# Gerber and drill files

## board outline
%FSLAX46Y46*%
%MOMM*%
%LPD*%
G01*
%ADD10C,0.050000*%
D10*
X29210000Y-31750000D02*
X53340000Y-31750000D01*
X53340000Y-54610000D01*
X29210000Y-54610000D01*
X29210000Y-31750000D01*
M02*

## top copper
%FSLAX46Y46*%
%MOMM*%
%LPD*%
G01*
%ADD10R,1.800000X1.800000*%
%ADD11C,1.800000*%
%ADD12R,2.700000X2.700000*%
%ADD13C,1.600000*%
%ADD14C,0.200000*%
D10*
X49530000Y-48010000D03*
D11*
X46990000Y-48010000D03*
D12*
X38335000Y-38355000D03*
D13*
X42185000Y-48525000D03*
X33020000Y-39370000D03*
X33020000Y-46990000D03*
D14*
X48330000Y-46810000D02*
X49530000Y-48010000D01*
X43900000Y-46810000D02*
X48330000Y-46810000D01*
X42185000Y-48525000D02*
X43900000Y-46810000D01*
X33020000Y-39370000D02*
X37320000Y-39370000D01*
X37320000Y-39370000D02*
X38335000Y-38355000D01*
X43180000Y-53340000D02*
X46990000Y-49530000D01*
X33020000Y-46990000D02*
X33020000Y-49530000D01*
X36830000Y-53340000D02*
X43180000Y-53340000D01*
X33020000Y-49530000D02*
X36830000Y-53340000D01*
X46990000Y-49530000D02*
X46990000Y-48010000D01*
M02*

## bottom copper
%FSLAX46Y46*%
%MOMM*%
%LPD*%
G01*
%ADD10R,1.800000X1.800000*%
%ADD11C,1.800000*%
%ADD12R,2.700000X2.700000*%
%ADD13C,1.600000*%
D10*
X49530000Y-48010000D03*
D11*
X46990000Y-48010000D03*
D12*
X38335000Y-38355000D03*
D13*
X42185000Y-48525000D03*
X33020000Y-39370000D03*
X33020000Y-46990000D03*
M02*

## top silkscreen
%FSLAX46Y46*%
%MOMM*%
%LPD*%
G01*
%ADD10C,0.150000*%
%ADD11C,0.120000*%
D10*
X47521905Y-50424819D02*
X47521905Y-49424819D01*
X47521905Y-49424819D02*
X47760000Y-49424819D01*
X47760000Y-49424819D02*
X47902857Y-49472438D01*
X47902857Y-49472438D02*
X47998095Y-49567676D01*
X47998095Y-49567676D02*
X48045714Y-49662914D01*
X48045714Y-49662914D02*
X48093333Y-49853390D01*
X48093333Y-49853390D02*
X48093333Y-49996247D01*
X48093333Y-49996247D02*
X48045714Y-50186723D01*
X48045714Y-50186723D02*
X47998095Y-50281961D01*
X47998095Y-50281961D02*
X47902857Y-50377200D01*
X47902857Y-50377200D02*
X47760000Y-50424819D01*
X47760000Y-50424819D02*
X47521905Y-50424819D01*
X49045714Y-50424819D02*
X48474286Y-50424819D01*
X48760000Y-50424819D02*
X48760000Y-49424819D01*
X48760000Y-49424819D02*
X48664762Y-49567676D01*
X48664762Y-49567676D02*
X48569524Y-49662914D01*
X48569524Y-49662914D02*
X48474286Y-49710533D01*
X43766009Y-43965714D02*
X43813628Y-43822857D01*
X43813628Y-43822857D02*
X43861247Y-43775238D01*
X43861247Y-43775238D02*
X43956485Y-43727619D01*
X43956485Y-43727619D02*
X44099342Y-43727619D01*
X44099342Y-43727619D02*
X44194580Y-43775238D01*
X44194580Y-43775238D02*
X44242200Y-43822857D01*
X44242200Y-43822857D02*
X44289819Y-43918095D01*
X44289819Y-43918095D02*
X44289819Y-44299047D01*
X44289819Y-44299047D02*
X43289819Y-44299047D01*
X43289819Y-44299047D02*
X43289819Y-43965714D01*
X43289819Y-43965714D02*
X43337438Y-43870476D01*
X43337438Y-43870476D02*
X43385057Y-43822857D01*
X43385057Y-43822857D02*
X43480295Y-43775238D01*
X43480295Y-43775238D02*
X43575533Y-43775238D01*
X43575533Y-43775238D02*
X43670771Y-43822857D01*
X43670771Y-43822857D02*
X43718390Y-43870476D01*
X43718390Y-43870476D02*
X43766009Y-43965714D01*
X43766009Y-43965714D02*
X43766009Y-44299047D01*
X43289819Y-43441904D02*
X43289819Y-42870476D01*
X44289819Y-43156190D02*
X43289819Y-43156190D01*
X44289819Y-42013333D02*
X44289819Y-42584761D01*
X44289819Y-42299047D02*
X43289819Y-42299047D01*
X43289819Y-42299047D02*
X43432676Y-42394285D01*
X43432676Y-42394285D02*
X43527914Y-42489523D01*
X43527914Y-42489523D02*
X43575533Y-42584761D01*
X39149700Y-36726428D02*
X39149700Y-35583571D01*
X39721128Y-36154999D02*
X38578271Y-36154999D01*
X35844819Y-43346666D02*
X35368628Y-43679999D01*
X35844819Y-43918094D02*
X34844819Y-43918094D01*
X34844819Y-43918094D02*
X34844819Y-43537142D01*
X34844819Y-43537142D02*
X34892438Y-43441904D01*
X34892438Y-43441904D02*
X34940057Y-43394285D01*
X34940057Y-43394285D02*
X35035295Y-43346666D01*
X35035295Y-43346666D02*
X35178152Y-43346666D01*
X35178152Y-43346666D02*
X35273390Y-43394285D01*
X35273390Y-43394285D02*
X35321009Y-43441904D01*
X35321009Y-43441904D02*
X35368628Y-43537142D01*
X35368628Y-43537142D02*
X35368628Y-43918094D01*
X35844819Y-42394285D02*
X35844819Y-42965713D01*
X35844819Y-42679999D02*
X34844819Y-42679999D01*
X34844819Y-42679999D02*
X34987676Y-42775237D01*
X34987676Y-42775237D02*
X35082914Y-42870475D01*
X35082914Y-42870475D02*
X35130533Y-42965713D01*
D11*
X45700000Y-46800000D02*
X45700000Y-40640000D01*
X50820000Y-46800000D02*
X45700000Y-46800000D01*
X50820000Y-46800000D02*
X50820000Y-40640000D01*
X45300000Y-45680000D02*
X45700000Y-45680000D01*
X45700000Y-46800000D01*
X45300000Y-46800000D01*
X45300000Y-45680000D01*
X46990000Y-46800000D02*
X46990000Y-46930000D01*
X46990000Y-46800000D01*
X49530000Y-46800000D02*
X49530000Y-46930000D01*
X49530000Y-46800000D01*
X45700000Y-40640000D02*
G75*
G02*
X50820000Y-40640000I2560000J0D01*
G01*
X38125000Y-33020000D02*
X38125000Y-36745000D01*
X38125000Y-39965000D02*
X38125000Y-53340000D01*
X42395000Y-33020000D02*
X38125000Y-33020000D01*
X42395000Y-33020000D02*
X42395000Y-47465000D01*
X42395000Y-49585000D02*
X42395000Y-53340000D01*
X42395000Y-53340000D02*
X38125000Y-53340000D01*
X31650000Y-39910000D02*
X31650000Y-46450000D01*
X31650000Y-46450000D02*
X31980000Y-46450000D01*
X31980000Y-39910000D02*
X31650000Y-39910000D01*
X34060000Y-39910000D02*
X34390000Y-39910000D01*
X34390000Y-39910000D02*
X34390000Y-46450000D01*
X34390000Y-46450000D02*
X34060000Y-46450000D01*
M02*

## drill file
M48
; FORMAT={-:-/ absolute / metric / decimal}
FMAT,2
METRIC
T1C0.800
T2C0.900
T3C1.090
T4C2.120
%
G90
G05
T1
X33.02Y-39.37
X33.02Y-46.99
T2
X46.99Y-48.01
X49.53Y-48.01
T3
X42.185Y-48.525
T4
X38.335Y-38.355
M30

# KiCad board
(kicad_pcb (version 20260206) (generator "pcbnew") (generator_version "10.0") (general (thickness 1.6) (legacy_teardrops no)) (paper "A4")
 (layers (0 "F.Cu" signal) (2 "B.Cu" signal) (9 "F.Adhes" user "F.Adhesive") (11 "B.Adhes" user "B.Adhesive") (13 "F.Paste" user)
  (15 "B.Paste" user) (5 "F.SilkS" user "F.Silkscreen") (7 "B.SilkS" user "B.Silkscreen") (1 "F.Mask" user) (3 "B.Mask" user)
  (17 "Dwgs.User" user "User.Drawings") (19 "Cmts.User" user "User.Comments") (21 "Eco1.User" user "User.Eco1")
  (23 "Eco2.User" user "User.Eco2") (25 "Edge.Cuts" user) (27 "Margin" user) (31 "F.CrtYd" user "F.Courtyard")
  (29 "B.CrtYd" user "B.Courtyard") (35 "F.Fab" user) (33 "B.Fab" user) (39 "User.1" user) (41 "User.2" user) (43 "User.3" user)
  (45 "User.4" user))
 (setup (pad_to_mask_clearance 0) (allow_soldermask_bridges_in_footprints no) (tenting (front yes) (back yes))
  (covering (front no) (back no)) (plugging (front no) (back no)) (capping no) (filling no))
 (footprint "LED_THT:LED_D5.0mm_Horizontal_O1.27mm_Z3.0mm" (layer "F.Cu") (at 49.53 48.01 180)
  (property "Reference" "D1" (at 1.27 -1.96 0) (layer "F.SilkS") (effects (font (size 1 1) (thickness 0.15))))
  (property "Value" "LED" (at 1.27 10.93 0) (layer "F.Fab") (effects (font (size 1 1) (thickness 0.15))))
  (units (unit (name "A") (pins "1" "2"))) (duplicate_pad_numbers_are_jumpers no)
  (fp_line (start 3.83 1.21) (end 3.83 7.37) (stroke (width 0.12) (type solid)) (layer "F.SilkS"))
  (fp_line (start -1.29 1.21) (end 3.83 1.21) (stroke (width 0.12) (type solid)) (layer "F.SilkS"))
  (fp_line (start -1.29 1.21) (end -1.29 7.37) (stroke (width 0.12) (type solid)) (layer "F.SilkS"))
  (fp_rect (start 3.83 1.21) (end 4.23 2.33) (stroke (width 0.12) (type solid)) (fill no) (layer "F.SilkS"))
  (fp_rect (start 2.54 1.08) (end 2.54 1.21) (stroke (width 0.12) (type solid)) (fill no) (layer "F.SilkS"))
  (fp_rect (start 0 1.08) (end 0 1.21) (stroke (width 0.12) (type solid)) (fill no) (layer "F.SilkS"))
  (fp_arc (start 3.83 7.37) (mid 1.27 9.93) (end -1.29 7.37) (stroke (width 0.12) (type solid)) (layer "F.SilkS"))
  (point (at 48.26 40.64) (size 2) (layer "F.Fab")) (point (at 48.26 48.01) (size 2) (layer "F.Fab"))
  (pad "1" thru_hole rect (at 0 0 180) (size 1.8 1.8) (drill 0.9) (layers "*.Cu" "*.Mask") (remove_unused_layers no) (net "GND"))
  (pad "2" thru_hole circle (at 2.54 0 180) (size 1.8 1.8) (drill 0.9) (layers "*.Cu" "*.Mask") (remove_unused_layers no) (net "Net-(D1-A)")))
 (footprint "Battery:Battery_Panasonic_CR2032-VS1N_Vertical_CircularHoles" (layer "F.Cu") (at 38.335 38.355 -90)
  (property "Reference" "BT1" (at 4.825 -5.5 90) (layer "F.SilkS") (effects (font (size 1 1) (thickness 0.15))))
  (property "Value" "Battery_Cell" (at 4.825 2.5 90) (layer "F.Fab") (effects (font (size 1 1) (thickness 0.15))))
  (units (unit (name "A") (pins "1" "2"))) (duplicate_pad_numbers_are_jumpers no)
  (fp_line (start -5.335 0.21) (end -1.61 0.21) (stroke (width 0.12) (type solid)) (layer "F.SilkS"))
  (fp_line (start 1.61 0.21) (end 14.985 0.21) (stroke (width 0.12) (type solid)) (layer "F.SilkS"))
  (fp_line (start -5.335 -4.06) (end -5.335 0.21) (stroke (width 0.12) (type solid)) (layer "F.SilkS"))
  (fp_line (start -5.335 -4.06) (end 9.11 -4.06) (stroke (width 0.12) (type solid)) (layer "F.SilkS"))
  (fp_line (start 11.23 -4.06) (end 14.985 -4.06) (stroke (width 0.12) (type solid)) (layer "F.SilkS"))
  (fp_line (start 14.985 -4.06) (end 14.985 0.21) (stroke (width 0.12) (type solid)) (layer "F.SilkS"))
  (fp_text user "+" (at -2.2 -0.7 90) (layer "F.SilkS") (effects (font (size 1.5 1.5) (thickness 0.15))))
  (pad "1" thru_hole rect (at 0 0) (size 2.7 2.7) (drill 2.12) (layers "*.Cu" "*.Mask") (remove_unused_layers no) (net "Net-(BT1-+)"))
  (pad "2" thru_hole circle (at 10.17 -3.85 270) (size 1.6 1.6) (drill 1.09) (layers "*.Cu" "*.Mask") (remove_unused_layers no) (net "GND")))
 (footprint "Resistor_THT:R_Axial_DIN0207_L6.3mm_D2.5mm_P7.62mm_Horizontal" (layer "F.Cu") (at 33.02 39.37 -90)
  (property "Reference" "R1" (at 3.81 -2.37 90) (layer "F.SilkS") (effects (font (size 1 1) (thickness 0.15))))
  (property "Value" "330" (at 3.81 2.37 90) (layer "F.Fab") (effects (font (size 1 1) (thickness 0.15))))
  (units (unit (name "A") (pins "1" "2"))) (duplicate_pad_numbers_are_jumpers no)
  (fp_line (start 0.54 1.37) (end 7.08 1.37) (stroke (width 0.12) (type solid)) (layer "F.SilkS"))
  (fp_line (start 7.08 1.37) (end 7.08 1.04) (stroke (width 0.12) (type solid)) (layer "F.SilkS"))
  (fp_line (start 0.54 1.04) (end 0.54 1.37) (stroke (width 0.12) (type solid)) (layer "F.SilkS"))
  (fp_line (start 0.54 -1.04) (end 0.54 -1.37) (stroke (width 0.12) (type solid)) (layer "F.SilkS"))
  (fp_line (start 0.54 -1.37) (end 7.08 -1.37) (stroke (width 0.12) (type solid)) (layer "F.SilkS"))
  (fp_line (start 7.08 -1.37) (end 7.08 -1.04) (stroke (width 0.12) (type solid)) (layer "F.SilkS"))
  (pad "1" thru_hole circle (at 0 0 270) (size 1.6 1.6) (drill 0.8) (layers "*.Cu" "*.Mask") (remove_unused_layers no) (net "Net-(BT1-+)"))
  (pad "2" thru_hole circle (at 7.62 0 270) (size 1.6 1.6) (drill 0.8) (layers "*.Cu" "*.Mask") (remove_unused_layers no) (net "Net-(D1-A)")))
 (gr_rect (start 29.21 31.75) (end 53.34 54.61) (stroke (width 0.05) (type default)) (fill no) (layer "Edge.Cuts"))
 (segment (start 48.33 46.81) (end 49.53 48.01) (width 0.2) (layer "F.Cu") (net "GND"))
 (segment (start 43.9 46.81) (end 48.33 46.81) (width 0.2) (layer "F.Cu") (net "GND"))
 (segment (start 42.185 48.525) (end 43.9 46.81) (width 0.2) (layer "F.Cu") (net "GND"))
 (segment (start 33.02 39.37) (end 37.32 39.37) (width 0.2) (layer "F.Cu") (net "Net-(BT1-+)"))
 (segment (start 37.32 39.37) (end 38.335 38.355) (width 0.2) (layer "F.Cu") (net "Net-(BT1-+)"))
 (segment (start 43.18 53.34) (end 46.99 49.53) (width 0.2) (layer "F.Cu") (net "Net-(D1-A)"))
 (segment (start 33.02 46.99) (end 33.02 49.53) (width 0.2) (layer "F.Cu") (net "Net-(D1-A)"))
 (segment (start 36.83 53.34) (end 43.18 53.34) (width 0.2) (layer "F.Cu") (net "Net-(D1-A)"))
 (segment (start 33.02 49.53) (end 36.83 53.34) (width 0.2) (layer "F.Cu") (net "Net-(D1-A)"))
 (segment (start 46.99 49.53) (end 46.99 48.01) (width 0.2) (layer "F.Cu") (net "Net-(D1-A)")))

